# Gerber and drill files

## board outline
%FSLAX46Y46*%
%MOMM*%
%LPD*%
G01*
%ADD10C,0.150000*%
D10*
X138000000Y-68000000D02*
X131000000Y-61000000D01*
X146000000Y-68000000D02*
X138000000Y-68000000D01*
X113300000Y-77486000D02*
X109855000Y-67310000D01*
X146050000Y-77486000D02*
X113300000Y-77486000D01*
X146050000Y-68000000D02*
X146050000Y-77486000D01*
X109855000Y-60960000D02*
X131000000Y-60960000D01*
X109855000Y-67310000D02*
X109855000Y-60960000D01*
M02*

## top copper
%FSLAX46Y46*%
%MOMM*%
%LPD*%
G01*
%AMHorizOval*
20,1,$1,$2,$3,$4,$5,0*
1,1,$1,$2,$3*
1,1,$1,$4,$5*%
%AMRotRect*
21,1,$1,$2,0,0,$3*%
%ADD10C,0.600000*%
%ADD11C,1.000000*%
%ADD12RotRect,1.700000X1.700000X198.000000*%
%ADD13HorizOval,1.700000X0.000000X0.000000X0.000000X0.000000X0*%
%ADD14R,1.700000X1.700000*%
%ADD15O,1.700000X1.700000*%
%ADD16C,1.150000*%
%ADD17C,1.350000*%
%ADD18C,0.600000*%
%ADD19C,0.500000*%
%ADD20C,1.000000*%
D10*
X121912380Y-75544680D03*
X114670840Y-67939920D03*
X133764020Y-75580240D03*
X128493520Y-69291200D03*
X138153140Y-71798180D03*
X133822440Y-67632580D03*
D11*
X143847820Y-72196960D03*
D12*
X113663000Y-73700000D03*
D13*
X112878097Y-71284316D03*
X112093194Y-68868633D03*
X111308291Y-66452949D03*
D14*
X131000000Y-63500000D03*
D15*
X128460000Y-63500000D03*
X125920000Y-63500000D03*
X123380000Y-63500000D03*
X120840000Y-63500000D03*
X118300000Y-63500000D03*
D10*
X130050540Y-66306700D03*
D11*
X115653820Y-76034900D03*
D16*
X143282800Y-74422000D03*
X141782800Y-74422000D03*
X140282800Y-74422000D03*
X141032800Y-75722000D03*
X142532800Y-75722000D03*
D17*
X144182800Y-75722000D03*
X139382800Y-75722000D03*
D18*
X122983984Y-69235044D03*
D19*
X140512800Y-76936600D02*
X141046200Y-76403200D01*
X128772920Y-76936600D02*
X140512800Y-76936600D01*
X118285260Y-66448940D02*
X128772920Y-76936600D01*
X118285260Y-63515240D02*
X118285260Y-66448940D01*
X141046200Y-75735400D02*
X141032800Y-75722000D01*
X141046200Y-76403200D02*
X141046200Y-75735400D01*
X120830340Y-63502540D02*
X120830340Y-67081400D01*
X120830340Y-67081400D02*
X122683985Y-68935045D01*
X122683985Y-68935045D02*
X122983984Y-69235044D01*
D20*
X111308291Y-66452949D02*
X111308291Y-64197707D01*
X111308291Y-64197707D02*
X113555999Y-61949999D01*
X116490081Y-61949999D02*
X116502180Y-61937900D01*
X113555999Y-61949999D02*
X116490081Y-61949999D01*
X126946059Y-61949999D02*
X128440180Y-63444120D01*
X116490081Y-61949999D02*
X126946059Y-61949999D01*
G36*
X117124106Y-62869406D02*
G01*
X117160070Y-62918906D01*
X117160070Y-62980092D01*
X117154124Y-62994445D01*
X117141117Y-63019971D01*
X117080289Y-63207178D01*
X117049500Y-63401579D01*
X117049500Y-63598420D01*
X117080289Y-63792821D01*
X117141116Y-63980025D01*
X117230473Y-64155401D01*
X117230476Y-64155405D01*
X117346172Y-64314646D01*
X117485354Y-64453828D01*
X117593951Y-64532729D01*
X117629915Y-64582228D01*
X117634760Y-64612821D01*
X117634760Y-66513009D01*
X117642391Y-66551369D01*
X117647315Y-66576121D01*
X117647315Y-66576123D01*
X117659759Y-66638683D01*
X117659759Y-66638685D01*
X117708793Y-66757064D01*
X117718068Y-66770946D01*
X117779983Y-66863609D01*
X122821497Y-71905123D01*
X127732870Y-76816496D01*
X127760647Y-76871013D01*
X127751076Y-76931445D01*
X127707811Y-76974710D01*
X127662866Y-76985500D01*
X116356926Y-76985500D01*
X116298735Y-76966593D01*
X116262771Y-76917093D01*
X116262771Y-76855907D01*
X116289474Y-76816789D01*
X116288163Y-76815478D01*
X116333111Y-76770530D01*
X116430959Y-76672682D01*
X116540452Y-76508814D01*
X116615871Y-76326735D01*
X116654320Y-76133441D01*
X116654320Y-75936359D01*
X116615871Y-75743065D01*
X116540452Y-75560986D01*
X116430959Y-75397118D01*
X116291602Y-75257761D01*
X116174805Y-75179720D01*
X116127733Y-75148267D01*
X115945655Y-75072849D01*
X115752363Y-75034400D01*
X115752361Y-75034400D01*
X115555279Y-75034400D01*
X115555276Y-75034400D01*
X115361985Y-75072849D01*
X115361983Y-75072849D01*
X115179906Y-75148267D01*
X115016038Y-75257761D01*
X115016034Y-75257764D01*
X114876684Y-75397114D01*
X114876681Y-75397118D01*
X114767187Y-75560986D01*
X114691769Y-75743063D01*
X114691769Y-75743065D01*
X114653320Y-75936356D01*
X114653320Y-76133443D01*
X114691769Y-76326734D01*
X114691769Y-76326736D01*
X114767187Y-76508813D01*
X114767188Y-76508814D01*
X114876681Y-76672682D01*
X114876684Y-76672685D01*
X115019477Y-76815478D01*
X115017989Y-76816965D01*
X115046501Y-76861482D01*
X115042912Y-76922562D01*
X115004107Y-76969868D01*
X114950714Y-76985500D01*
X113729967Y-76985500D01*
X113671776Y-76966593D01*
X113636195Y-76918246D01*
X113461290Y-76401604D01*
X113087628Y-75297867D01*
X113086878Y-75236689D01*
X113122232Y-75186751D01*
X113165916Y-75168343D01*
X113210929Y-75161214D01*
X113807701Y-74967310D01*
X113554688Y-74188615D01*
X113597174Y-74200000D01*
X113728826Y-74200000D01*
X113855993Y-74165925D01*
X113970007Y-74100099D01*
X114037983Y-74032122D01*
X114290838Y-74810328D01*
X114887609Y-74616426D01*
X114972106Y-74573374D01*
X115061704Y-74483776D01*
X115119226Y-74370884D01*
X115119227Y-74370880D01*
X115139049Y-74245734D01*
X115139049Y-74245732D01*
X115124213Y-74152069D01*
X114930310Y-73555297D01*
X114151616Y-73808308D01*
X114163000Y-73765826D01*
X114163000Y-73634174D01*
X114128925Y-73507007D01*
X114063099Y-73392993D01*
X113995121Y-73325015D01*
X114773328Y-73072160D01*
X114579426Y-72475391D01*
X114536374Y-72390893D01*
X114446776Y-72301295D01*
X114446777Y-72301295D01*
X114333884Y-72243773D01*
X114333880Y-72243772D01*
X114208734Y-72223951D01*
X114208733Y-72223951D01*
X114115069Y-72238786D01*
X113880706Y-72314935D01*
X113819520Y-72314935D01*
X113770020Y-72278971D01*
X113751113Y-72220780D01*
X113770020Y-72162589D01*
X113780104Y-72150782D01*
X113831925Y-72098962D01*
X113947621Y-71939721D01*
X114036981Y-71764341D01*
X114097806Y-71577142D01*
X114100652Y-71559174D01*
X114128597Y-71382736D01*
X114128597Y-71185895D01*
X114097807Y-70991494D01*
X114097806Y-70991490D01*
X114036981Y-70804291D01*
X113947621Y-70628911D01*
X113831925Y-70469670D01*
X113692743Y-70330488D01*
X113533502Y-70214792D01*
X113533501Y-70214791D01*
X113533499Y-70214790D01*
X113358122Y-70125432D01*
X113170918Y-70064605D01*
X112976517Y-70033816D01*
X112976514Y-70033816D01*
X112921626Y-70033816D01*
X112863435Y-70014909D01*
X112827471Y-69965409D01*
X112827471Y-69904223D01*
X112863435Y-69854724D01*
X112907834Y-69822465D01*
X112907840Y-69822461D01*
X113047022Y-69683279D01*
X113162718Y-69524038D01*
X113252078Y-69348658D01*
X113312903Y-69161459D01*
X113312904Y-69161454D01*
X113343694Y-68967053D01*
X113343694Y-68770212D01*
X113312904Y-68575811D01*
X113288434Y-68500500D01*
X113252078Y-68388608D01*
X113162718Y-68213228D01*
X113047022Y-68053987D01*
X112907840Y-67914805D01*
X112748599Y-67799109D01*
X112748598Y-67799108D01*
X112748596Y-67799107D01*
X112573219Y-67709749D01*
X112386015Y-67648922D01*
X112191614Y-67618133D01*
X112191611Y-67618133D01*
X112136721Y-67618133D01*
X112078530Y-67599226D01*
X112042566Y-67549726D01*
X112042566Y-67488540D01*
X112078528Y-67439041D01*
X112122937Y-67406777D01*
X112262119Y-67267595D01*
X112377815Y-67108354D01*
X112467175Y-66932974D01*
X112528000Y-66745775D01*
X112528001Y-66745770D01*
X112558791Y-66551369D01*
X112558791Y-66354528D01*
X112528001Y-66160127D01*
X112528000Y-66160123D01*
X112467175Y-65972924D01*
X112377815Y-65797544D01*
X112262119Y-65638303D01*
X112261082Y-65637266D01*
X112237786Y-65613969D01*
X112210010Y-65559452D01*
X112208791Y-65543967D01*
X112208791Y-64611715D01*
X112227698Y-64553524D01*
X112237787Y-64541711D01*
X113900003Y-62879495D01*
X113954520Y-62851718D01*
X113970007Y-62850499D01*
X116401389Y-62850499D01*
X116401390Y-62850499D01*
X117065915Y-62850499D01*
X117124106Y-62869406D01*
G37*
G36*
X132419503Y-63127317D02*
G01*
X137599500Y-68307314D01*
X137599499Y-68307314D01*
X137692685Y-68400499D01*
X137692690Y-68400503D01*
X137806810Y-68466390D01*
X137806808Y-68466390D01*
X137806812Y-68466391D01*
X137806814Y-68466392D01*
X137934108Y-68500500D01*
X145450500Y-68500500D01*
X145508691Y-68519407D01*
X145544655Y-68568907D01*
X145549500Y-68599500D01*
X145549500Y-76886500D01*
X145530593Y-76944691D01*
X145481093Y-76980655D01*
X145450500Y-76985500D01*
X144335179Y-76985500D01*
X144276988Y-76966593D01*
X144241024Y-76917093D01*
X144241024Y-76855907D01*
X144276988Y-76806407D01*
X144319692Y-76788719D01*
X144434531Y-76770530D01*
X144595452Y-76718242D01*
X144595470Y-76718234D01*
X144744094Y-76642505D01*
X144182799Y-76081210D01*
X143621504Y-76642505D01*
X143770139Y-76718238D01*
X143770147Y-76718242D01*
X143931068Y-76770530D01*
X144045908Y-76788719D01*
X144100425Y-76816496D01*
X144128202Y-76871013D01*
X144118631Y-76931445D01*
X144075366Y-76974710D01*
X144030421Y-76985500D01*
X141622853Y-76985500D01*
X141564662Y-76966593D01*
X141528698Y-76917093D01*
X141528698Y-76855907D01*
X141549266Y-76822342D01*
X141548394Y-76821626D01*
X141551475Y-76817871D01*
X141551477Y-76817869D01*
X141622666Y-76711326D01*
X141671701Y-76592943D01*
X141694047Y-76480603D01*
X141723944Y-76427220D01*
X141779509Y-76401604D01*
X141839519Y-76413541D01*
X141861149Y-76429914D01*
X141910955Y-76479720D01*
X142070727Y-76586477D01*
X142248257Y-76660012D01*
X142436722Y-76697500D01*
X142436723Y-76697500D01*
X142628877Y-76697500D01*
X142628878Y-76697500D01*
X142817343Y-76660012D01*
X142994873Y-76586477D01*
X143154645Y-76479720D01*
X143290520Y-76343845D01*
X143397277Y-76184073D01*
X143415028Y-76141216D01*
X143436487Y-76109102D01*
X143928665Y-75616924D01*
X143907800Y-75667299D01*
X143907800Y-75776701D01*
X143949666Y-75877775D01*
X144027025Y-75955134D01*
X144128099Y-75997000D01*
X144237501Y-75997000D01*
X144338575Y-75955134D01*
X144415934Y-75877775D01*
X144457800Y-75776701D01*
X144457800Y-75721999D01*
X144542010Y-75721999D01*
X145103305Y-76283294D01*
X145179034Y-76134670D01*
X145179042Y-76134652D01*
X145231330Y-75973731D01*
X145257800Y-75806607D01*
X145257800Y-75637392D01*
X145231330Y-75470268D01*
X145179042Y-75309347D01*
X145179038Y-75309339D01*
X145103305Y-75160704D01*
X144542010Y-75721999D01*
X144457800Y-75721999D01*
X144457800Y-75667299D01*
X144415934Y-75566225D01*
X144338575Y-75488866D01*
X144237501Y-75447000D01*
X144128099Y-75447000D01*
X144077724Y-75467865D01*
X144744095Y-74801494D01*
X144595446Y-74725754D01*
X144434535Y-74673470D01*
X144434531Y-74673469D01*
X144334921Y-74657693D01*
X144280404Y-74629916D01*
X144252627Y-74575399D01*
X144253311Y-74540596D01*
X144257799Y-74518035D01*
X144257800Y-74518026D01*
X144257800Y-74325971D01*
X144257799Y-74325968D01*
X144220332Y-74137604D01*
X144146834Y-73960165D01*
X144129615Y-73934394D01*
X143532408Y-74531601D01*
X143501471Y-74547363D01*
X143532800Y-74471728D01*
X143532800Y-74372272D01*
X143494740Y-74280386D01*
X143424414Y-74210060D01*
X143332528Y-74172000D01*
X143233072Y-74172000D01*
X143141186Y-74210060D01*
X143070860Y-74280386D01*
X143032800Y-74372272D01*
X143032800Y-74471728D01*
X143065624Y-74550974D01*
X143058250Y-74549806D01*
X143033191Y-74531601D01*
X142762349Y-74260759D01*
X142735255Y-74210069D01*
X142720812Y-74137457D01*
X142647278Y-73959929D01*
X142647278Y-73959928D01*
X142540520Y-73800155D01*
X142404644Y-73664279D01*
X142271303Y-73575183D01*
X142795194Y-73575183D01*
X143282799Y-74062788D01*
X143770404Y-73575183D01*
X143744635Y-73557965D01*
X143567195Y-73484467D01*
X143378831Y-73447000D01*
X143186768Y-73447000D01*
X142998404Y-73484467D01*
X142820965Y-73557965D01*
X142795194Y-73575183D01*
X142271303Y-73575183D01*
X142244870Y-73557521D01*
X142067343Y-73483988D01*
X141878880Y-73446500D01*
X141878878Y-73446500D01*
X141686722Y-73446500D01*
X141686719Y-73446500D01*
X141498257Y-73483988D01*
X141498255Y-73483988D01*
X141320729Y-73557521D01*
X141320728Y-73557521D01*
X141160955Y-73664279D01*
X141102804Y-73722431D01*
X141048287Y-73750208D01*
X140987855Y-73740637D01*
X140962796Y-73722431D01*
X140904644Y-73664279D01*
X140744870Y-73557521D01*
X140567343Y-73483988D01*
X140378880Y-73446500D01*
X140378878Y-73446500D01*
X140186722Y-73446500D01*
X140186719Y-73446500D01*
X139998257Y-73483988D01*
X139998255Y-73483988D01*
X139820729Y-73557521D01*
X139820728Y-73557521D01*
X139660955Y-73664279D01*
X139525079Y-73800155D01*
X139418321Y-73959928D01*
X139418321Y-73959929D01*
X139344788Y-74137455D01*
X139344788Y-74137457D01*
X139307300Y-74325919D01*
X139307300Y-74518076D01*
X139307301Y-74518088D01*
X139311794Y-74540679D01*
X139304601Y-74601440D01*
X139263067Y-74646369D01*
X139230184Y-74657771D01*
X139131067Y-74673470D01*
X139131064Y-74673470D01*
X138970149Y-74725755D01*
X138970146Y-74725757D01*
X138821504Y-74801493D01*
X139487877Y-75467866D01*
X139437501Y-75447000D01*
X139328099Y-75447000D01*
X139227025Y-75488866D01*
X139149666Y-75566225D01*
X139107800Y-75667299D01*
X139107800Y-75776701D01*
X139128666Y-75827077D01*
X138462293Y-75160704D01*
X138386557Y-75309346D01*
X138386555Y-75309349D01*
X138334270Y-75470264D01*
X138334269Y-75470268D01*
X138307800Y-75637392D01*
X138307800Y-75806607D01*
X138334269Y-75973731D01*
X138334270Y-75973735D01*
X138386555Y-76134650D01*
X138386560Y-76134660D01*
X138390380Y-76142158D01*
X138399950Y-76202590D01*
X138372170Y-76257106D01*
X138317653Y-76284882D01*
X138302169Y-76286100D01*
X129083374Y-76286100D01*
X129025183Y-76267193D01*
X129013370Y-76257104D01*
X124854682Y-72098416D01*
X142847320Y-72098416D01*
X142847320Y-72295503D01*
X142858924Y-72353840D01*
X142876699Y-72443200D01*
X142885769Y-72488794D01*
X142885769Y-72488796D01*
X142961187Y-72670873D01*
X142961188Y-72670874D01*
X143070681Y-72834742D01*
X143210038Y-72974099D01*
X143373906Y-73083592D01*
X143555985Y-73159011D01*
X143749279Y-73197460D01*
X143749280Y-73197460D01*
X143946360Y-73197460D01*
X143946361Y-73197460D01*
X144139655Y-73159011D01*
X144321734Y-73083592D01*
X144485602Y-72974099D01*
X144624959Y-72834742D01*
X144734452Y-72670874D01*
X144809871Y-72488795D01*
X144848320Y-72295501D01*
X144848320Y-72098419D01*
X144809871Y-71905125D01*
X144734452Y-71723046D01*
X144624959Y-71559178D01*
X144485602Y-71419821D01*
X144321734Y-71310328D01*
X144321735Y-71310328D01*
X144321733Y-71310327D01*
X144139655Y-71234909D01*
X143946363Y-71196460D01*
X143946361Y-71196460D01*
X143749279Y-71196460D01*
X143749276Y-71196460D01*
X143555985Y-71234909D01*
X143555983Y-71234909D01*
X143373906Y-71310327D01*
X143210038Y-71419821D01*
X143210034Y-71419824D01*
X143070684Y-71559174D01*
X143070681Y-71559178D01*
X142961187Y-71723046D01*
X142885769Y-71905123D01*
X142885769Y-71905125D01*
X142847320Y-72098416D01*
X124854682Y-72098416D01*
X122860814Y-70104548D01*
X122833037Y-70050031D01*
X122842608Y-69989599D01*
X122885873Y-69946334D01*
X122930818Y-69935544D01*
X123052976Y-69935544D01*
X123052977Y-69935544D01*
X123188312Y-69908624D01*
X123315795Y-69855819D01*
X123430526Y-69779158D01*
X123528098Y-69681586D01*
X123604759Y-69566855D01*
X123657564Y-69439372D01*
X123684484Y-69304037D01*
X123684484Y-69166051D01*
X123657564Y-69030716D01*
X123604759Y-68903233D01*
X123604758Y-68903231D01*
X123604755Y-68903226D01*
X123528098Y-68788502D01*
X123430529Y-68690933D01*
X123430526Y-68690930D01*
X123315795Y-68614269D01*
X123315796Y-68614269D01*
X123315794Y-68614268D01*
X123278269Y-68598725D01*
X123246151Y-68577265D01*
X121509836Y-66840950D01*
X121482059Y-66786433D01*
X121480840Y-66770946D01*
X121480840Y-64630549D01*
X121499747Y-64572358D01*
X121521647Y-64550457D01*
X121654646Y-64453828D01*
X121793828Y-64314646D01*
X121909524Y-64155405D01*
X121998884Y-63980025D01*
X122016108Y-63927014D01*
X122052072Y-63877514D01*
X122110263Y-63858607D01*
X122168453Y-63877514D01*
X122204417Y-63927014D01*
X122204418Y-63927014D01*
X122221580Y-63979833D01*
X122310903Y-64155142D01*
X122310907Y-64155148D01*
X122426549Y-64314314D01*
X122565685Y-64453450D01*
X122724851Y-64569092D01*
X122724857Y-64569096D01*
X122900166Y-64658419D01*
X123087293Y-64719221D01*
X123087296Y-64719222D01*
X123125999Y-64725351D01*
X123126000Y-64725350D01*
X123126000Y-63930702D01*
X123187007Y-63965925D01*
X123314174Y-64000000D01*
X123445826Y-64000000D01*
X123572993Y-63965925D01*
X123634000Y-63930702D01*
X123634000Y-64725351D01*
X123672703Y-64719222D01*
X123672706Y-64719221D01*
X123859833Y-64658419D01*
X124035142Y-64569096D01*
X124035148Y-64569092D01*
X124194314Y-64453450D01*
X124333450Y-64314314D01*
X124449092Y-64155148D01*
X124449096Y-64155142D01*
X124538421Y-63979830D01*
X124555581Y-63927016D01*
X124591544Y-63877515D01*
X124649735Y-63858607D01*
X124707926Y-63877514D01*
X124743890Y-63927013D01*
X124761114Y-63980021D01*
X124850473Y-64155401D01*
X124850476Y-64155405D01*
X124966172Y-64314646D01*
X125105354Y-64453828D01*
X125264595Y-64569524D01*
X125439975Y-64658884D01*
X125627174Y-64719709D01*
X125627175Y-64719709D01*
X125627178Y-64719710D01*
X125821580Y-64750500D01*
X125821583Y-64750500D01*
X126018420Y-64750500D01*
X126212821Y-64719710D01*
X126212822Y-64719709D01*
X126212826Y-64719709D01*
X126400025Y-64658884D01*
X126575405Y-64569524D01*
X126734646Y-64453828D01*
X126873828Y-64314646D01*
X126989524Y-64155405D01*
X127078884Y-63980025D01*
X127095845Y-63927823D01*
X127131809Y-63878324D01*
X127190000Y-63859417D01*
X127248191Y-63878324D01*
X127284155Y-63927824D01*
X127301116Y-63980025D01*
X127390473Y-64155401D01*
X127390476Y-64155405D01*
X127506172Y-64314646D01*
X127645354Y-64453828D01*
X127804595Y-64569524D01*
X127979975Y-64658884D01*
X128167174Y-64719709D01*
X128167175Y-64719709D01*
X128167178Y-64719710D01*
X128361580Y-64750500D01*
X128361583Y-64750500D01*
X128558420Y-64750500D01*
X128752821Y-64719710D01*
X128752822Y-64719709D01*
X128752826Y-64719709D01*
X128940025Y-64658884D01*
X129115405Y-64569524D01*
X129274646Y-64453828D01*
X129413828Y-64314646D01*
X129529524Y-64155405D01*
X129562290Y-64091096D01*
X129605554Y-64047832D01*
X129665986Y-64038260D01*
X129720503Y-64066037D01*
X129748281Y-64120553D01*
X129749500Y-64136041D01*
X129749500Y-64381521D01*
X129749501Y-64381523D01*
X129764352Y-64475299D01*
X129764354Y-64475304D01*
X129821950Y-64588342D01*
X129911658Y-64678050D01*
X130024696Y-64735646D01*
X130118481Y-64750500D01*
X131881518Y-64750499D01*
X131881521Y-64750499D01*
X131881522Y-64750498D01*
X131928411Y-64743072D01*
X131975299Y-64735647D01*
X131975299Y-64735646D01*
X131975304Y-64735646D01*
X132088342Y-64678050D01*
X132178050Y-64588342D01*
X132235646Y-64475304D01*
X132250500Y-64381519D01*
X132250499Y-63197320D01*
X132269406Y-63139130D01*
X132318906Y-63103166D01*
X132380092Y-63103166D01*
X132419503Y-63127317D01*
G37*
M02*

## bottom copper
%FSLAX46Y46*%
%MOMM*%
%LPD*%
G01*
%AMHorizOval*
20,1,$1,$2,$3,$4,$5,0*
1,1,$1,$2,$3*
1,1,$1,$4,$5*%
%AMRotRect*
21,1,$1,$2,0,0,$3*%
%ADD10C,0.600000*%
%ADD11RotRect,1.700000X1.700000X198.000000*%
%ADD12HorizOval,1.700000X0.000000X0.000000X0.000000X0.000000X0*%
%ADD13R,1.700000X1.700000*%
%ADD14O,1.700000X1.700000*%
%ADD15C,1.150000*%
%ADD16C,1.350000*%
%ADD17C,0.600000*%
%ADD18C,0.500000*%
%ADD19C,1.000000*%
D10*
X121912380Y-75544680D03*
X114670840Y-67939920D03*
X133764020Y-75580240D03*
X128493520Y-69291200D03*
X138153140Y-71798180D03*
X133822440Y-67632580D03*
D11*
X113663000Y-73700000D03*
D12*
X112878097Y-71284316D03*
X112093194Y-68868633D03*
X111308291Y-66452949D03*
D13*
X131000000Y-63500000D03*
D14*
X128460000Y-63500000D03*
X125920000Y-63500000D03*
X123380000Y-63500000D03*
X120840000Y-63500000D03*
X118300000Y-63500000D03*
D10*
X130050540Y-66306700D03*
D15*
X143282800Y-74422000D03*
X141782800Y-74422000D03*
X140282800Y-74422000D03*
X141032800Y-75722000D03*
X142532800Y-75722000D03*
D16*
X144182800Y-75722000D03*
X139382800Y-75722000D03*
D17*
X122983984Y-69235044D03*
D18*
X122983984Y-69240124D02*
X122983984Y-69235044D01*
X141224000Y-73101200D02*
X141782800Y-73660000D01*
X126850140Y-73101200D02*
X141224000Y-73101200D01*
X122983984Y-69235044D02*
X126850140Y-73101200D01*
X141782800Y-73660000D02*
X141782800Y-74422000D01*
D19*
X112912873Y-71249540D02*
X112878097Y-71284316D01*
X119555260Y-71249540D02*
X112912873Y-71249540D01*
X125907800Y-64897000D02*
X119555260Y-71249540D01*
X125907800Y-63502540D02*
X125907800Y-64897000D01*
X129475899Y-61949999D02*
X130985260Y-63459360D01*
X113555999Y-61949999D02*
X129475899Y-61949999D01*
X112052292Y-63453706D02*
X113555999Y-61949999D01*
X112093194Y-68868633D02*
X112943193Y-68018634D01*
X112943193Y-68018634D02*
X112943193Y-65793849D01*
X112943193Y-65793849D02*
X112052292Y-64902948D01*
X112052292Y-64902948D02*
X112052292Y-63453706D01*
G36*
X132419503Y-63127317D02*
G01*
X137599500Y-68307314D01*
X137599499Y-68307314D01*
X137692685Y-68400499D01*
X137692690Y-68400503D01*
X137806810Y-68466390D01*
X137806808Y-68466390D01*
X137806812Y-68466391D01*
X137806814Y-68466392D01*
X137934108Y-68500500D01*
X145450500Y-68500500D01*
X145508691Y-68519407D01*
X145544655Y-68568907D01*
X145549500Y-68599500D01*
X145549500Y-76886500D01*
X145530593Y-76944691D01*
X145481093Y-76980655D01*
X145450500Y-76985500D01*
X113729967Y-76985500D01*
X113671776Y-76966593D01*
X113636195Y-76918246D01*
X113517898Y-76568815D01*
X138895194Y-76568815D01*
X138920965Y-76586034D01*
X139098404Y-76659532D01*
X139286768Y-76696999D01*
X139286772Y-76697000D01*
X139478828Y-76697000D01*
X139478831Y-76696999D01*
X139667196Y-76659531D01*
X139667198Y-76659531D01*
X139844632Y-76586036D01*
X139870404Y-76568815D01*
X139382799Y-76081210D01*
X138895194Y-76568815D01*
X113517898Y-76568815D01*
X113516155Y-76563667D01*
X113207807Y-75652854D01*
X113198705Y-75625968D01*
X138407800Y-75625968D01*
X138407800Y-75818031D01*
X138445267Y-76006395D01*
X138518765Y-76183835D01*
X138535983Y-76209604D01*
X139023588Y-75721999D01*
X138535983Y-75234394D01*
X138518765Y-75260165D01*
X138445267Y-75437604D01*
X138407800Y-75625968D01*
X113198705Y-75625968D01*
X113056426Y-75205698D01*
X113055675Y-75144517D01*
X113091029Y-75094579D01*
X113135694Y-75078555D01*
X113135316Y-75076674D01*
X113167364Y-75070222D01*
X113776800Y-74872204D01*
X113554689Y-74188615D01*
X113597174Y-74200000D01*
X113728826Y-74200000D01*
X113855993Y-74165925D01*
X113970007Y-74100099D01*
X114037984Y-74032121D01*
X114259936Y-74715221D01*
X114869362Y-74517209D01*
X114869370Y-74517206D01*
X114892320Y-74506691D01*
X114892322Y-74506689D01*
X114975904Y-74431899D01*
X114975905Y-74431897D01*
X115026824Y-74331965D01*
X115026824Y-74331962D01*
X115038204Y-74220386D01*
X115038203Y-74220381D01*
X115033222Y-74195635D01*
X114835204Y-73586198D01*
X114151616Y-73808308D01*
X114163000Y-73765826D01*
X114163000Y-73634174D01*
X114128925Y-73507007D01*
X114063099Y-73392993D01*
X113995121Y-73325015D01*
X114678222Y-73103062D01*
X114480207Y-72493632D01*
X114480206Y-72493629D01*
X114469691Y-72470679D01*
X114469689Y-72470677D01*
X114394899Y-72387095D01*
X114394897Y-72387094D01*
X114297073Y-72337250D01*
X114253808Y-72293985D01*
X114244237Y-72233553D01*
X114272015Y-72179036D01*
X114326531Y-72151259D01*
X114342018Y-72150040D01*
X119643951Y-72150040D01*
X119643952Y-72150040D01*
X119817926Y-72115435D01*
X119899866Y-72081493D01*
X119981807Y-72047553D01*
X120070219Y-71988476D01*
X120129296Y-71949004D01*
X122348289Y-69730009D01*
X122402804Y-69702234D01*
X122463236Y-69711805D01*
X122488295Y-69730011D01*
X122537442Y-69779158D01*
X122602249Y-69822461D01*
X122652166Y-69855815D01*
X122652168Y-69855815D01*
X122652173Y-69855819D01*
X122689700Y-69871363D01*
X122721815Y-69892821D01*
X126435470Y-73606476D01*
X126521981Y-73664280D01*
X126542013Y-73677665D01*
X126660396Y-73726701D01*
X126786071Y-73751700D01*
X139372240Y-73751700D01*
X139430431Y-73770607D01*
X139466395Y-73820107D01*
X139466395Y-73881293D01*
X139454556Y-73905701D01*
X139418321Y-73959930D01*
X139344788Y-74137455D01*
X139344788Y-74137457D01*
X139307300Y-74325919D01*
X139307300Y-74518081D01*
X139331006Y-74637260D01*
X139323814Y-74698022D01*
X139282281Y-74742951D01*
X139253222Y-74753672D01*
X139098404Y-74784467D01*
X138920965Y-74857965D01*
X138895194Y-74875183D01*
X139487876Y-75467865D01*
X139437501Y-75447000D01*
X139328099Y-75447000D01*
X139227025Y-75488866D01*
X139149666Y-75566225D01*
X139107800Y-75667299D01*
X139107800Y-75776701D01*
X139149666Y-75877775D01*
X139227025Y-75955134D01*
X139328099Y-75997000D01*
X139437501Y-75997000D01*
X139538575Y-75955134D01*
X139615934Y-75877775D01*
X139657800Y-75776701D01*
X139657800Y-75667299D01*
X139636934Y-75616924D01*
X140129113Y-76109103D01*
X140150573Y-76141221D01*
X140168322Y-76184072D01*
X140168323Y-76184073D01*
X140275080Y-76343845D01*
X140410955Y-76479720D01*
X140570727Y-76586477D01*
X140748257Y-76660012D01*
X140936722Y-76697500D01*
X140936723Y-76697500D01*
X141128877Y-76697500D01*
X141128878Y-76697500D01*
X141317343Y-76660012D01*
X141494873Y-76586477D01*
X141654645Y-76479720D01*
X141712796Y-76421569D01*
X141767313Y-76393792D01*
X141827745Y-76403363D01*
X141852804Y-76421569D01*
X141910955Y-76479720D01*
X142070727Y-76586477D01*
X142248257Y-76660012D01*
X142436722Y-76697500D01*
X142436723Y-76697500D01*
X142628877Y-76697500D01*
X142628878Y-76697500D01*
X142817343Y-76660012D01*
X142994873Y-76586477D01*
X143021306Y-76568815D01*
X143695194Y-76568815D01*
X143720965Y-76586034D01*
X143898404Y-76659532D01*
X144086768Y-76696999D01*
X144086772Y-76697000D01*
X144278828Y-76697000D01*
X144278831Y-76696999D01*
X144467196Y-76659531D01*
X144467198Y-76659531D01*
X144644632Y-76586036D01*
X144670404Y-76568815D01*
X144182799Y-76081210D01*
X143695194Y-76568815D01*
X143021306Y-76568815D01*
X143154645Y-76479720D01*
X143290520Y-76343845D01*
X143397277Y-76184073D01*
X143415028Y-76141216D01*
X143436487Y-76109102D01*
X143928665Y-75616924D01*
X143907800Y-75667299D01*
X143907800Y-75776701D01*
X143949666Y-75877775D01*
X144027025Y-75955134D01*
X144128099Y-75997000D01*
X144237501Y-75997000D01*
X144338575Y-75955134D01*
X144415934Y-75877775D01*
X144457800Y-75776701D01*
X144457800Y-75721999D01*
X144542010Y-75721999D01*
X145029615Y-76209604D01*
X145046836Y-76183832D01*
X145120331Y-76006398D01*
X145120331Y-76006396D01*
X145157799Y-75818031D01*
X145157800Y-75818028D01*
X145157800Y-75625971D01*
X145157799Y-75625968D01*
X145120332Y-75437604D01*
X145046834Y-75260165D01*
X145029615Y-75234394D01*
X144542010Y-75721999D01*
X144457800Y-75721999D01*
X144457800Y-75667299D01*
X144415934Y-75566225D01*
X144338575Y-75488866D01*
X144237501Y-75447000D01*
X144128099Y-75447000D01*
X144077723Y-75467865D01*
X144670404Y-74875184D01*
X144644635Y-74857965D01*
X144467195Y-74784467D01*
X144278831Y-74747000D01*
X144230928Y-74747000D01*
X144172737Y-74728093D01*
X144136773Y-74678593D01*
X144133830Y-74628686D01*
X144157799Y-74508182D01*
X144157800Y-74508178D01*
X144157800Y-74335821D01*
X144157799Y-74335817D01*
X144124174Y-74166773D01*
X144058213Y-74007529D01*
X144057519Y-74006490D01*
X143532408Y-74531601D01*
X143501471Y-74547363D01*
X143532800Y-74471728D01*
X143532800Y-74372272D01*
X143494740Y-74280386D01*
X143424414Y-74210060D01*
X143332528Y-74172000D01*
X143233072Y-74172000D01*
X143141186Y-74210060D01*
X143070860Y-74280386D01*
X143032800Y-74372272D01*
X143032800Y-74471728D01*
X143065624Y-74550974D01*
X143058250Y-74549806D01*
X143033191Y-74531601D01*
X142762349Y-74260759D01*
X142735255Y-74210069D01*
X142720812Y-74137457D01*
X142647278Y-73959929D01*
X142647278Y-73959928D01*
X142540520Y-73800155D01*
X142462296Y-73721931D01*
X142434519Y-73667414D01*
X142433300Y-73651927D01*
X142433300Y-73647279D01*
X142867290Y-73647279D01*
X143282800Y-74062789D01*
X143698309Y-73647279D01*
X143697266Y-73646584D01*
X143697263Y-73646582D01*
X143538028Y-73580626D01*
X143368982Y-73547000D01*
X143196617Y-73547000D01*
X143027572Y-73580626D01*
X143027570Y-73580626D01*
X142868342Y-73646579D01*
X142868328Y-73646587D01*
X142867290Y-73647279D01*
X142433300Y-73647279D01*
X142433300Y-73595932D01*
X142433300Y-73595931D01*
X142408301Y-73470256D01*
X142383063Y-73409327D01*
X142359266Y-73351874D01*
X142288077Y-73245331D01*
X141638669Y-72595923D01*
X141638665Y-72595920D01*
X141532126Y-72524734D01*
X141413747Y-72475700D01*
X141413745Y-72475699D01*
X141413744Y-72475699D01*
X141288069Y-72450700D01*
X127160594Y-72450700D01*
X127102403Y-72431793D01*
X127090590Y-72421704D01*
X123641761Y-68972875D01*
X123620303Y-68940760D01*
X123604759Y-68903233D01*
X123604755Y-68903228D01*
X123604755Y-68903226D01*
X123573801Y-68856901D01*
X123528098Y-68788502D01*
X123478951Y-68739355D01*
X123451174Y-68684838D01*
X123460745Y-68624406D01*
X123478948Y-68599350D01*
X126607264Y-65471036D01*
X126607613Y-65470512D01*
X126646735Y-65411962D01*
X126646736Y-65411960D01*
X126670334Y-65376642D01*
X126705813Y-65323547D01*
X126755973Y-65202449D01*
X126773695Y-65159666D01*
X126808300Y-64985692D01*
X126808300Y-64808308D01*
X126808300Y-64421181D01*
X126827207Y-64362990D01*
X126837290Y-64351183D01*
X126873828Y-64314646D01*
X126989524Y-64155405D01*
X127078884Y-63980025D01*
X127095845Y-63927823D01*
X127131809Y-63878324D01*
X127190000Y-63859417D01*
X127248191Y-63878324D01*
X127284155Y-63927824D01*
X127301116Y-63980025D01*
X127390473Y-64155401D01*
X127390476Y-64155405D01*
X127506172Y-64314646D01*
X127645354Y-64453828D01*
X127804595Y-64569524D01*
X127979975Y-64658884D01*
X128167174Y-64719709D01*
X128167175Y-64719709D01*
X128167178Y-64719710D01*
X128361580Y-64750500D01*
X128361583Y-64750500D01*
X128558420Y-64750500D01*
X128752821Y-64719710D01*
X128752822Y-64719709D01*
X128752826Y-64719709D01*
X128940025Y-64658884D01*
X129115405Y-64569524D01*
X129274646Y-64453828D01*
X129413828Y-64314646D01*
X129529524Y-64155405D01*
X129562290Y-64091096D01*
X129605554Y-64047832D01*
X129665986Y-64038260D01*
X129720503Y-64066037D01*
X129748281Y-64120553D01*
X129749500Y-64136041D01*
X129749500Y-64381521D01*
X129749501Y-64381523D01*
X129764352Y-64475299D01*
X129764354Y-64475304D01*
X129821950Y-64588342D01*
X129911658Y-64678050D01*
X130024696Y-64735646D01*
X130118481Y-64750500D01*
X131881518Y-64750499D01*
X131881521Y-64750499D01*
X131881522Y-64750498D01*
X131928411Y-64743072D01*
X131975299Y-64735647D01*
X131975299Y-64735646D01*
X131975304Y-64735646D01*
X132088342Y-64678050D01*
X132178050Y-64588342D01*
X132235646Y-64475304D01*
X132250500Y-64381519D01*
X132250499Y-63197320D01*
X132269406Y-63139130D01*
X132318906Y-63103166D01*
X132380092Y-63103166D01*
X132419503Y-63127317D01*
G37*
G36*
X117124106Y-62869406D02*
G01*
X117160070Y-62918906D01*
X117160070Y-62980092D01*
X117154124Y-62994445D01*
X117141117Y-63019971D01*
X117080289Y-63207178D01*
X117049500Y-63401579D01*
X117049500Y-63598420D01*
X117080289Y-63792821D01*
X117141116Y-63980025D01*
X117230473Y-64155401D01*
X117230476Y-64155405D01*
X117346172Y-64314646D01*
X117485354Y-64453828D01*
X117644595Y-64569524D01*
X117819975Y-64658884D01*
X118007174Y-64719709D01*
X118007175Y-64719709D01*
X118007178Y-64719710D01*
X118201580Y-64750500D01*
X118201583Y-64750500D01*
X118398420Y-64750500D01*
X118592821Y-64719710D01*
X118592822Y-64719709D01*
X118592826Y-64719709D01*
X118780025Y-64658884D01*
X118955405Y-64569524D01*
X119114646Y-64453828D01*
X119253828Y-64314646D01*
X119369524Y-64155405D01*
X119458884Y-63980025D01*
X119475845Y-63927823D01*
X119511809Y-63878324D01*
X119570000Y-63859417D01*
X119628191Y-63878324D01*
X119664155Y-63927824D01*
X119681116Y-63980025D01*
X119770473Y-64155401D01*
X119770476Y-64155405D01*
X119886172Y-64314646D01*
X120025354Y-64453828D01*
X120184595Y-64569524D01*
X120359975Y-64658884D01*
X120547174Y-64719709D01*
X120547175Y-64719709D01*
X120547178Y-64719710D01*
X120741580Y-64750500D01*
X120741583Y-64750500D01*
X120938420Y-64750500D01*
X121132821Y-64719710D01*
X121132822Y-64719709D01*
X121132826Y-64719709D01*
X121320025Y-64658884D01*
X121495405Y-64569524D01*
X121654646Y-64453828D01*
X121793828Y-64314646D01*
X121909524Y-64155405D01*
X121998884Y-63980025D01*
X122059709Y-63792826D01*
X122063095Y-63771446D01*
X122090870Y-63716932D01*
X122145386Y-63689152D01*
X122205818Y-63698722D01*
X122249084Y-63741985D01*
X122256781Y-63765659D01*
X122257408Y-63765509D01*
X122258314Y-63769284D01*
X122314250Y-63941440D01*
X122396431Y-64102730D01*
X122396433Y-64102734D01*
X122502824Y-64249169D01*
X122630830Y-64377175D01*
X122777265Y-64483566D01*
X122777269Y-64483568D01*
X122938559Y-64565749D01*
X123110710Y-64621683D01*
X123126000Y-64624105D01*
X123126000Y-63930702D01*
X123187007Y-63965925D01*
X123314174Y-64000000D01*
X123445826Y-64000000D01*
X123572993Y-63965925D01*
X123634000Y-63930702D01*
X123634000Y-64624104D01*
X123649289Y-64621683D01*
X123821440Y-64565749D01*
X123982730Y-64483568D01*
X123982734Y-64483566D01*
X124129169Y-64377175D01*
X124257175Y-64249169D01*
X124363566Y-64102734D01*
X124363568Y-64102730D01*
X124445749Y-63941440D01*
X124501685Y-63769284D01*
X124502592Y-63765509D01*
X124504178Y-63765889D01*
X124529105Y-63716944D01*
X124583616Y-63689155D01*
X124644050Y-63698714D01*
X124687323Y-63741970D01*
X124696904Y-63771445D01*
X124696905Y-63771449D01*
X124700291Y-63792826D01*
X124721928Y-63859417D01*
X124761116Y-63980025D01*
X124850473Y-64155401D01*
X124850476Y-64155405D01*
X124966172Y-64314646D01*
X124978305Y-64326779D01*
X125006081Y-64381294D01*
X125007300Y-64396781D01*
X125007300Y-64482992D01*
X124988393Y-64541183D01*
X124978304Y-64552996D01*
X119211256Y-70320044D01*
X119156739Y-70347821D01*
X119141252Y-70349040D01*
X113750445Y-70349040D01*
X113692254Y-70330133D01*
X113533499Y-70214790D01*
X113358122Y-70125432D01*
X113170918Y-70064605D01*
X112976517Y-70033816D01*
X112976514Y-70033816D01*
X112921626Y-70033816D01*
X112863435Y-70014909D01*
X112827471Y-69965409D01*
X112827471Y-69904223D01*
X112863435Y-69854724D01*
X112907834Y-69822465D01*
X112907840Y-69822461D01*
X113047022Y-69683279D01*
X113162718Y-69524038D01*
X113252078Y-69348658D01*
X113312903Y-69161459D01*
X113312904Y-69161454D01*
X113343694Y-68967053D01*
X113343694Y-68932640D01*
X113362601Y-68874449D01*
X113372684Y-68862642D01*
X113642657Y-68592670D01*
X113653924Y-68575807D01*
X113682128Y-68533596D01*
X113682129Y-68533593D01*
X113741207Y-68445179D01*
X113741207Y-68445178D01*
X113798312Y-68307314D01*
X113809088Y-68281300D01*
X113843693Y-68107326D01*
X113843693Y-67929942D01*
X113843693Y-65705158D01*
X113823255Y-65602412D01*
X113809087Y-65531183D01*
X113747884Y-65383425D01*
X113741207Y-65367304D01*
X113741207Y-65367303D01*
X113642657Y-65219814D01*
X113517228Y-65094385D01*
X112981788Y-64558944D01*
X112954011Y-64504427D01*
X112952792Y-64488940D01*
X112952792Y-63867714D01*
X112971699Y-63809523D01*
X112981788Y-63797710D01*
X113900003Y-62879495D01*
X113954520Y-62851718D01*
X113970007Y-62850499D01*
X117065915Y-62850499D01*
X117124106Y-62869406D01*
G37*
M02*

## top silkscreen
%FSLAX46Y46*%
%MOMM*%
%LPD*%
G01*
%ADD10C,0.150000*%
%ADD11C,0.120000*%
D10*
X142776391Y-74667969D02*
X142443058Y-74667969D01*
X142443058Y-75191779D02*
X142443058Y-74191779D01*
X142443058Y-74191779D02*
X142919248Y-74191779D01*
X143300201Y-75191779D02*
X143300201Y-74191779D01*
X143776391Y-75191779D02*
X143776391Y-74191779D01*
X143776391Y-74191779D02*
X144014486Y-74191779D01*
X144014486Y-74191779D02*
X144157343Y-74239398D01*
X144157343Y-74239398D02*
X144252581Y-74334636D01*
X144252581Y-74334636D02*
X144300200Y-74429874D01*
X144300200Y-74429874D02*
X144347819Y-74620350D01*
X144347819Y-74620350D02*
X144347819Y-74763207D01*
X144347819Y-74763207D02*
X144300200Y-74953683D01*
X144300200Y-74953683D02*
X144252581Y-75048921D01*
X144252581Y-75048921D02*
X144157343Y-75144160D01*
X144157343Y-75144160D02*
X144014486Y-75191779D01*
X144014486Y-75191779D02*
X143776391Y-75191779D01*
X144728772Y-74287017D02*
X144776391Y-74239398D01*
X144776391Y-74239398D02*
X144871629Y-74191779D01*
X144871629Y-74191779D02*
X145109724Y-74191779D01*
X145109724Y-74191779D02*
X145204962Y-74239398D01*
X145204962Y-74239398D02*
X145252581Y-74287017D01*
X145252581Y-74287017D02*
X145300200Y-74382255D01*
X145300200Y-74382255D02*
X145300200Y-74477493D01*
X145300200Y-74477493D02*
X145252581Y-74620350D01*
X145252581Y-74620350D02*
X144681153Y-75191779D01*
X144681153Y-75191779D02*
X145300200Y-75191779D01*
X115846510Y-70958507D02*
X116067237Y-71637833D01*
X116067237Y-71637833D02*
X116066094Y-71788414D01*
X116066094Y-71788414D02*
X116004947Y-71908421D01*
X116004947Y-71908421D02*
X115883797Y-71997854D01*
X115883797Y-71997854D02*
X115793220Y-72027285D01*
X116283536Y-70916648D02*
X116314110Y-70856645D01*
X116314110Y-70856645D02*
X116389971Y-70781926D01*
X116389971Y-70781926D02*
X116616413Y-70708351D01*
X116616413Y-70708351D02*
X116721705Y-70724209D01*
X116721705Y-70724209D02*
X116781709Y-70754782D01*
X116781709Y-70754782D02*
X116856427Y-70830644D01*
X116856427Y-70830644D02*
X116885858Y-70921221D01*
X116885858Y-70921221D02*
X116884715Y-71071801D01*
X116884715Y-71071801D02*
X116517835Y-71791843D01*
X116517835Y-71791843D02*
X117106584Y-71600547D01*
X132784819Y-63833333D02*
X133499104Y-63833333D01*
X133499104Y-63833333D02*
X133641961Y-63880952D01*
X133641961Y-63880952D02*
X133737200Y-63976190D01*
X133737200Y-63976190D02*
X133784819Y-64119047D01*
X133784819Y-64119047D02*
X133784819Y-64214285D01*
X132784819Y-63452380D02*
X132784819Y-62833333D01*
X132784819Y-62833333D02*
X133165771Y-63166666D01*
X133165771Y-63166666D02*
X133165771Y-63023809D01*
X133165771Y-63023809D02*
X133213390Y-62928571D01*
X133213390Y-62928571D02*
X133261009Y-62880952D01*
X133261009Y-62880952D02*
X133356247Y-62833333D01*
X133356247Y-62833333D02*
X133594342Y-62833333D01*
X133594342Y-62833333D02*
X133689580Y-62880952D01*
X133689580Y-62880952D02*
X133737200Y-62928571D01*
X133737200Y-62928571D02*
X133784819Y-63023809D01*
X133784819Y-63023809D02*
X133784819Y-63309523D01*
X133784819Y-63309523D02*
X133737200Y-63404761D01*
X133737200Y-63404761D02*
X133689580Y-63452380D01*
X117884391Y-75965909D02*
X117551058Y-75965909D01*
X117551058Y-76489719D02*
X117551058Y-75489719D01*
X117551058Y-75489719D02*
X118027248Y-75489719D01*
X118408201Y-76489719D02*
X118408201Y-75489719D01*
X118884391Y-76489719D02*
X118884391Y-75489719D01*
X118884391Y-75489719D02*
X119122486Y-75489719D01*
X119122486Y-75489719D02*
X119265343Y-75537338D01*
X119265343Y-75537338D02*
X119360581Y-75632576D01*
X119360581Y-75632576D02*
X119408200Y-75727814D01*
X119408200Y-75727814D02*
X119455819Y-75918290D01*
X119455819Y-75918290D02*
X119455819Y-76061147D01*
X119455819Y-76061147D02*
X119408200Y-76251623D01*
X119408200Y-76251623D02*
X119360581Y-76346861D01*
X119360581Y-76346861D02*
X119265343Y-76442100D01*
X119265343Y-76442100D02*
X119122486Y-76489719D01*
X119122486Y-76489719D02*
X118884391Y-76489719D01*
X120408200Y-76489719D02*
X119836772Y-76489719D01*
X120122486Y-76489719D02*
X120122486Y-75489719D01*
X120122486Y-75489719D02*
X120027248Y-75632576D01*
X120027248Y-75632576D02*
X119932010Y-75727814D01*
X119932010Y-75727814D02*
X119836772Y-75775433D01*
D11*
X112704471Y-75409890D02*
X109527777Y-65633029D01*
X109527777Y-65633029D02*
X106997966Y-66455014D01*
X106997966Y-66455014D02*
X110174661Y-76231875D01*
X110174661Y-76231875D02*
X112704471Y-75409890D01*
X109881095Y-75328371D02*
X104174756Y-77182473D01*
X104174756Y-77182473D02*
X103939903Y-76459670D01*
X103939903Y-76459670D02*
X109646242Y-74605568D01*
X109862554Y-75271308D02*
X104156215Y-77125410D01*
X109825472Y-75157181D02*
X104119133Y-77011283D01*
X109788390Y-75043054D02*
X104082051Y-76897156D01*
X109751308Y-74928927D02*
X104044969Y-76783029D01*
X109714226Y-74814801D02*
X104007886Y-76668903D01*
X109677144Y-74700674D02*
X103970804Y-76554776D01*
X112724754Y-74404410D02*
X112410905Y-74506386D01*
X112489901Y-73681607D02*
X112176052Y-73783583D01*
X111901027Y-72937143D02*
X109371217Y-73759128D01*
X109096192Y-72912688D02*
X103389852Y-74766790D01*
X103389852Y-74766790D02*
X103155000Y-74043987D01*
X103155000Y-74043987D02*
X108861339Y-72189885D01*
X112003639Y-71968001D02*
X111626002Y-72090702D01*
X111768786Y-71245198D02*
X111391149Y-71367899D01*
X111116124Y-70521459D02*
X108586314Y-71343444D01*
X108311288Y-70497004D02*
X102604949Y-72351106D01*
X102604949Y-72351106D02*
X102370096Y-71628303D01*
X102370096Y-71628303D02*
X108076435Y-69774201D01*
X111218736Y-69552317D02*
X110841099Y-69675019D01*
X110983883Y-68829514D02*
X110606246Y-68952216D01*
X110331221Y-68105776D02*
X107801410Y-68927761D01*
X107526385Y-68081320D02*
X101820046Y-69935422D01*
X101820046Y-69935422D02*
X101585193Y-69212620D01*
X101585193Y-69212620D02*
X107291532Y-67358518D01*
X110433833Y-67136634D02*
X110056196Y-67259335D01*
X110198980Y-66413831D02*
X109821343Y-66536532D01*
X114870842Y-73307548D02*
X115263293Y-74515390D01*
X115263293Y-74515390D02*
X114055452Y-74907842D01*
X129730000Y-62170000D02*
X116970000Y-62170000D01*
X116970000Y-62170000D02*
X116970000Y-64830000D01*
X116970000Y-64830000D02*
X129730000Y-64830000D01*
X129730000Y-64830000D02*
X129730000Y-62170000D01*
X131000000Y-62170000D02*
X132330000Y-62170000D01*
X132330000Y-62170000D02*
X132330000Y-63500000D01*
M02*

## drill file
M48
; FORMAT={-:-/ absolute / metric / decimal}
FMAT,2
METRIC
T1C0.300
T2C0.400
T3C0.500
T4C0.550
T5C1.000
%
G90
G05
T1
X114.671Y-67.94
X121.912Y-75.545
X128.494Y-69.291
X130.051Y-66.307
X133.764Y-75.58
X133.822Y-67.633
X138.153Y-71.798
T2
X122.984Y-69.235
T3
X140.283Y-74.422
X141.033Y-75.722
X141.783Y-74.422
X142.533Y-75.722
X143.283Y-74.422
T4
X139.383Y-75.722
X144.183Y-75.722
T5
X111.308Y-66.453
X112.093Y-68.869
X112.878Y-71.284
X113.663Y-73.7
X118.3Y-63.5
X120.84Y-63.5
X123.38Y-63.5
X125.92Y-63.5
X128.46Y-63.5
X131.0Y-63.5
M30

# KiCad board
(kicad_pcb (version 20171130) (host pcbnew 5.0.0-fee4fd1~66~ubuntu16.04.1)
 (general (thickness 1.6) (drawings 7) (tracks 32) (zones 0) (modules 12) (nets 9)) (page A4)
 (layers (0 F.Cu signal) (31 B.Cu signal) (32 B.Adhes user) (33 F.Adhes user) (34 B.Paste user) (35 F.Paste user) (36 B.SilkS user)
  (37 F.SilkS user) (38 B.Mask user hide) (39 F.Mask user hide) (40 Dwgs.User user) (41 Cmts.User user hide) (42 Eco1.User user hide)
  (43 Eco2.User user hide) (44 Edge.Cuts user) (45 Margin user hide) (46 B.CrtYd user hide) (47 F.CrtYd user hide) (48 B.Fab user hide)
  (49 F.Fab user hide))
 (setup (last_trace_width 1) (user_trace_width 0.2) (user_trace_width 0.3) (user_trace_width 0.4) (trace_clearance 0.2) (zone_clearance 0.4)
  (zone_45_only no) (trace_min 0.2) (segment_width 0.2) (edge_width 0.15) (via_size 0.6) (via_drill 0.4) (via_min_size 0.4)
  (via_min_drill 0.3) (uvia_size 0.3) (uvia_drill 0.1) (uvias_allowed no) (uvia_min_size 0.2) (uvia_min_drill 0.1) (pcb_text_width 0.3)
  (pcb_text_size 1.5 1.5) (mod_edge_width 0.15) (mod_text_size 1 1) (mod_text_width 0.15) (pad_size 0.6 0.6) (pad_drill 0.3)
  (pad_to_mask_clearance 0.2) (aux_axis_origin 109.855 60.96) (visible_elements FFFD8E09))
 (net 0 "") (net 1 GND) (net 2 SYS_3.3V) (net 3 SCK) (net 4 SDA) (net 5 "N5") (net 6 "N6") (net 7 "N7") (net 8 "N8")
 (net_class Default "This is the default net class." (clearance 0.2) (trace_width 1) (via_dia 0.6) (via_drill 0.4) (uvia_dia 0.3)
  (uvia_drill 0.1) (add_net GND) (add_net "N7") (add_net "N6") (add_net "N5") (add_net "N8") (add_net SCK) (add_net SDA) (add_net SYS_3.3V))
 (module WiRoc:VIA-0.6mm (layer F.Cu) (at 121.91238 75.54468)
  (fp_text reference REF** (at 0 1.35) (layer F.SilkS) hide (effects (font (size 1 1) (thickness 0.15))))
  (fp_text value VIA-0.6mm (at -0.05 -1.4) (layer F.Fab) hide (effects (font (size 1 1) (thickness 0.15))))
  (pad 1 thru_hole circle (at 0 0) (size 0.6 0.6) (drill 0.3) (layers *.Cu) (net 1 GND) (zone_connect 2)))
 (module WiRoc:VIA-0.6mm (layer F.Cu) (at 114.67084 67.93992)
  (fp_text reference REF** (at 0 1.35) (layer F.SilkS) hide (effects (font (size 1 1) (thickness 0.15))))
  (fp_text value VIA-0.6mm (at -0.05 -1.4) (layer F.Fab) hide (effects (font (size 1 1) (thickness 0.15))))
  (pad 1 thru_hole circle (at 0 0) (size 0.6 0.6) (drill 0.3) (layers *.Cu) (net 1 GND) (zone_connect 2)))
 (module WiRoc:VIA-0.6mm (layer F.Cu) (at 133.76402 75.58024)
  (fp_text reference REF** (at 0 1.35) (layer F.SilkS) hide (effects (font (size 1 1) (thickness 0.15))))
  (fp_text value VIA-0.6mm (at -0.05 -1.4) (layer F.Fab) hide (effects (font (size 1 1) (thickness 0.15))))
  (pad 1 thru_hole circle (at 0 0) (size 0.6 0.6) (drill 0.3) (layers *.Cu) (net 1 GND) (zone_connect 2)))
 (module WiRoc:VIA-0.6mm (layer F.Cu) (at 128.49352 69.2912)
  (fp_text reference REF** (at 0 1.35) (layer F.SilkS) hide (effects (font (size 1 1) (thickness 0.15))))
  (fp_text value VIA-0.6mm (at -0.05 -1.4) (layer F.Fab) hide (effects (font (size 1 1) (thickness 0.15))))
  (pad 1 thru_hole circle (at 0 0) (size 0.6 0.6) (drill 0.3) (layers *.Cu) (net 1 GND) (zone_connect 2)))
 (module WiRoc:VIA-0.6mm (layer F.Cu) (at 138.15314 71.79818)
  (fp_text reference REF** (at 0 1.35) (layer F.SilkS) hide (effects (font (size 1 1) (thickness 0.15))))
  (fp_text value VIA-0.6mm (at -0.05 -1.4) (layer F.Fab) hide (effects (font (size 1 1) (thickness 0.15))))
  (pad 1 thru_hole circle (at 0 0) (size 0.6 0.6) (drill 0.3) (layers *.Cu) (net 1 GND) (zone_connect 2)))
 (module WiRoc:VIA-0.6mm (layer F.Cu) (at 133.82244 67.63258)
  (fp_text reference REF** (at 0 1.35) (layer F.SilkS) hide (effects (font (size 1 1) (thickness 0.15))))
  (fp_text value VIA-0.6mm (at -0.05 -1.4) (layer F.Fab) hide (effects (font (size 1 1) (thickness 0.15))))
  (pad 1 thru_hole circle (at 0 0) (size 0.6 0.6) (drill 0.3) (layers *.Cu) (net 1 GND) (zone_connect 2)))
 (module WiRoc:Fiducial (layer F.Cu) (at 143.84782 72.19696)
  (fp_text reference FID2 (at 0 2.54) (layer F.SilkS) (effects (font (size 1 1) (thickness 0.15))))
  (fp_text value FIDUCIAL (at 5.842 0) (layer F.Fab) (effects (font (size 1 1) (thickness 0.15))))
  (pad 1 smd circle (at 0 0) (size 1 1) (layers F.Cu F.Mask) (solder_mask_margin 0.5) (clearance 0.5)))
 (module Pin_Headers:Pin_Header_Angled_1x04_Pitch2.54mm (layer F.Cu) (at 113.663 73.7 198)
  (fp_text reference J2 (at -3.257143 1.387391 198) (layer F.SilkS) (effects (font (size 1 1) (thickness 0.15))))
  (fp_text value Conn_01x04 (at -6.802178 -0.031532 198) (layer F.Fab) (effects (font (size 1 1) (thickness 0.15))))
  (fp_line (start 1.44 -1.33) (end 1.44 8.95) (layer F.SilkS) (width 0.12))
  (fp_line (start 1.44 8.95) (end 4.1 8.95) (layer F.SilkS) (width 0.12))
  (fp_line (start 4.1 8.95) (end 4.1 -1.33) (layer F.SilkS) (width 0.12))
  (fp_line (start 4.1 -1.33) (end 1.44 -1.33) (layer F.SilkS) (width 0.12))
  (fp_line (start 4.1 -0.38) (end 10.1 -0.38) (layer F.SilkS) (width 0.12))
  (fp_line (start 10.1 -0.38) (end 10.1 0.38) (layer F.SilkS) (width 0.12))
  (fp_line (start 10.1 0.38) (end 4.1 0.38) (layer F.SilkS) (width 0.12))
  (fp_line (start 4.1 -0.32) (end 10.1 -0.32) (layer F.SilkS) (width 0.12))
  (fp_line (start 4.1 -0.2) (end 10.1 -0.2) (layer F.SilkS) (width 0.12))
  (fp_line (start 4.1 -0.08) (end 10.1 -0.08) (layer F.SilkS) (width 0.12))
  (fp_line (start 4.1 0.04) (end 10.1 0.04) (layer F.SilkS) (width 0.12))
  (fp_line (start 4.1 0.16) (end 10.1 0.16) (layer F.SilkS) (width 0.12))
  (fp_line (start 4.1 0.28) (end 10.1 0.28) (layer F.SilkS) (width 0.12))
  (fp_line (start 1.11 -0.38) (end 1.44 -0.38) (layer F.SilkS) (width 0.12))
  (fp_line (start 1.11 0.38) (end 1.44 0.38) (layer F.SilkS) (width 0.12))
  (fp_line (start 1.44 1.27) (end 4.1 1.27) (layer F.SilkS) (width 0.12))
  (fp_line (start 4.1 2.16) (end 10.1 2.16) (layer F.SilkS) (width 0.12))
  (fp_line (start 10.1 2.16) (end 10.1 2.92) (layer F.SilkS) (width 0.12))
  (fp_line (start 10.1 2.92) (end 4.1 2.92) (layer F.SilkS) (width 0.12))
  (fp_line (start 1.042929 2.16) (end 1.44 2.16) (layer F.SilkS) (width 0.12))
  (fp_line (start 1.042929 2.92) (end 1.44 2.92) (layer F.SilkS) (width 0.12))
  (fp_line (start 1.44 3.81) (end 4.1 3.81) (layer F.SilkS) (width 0.12))
  (fp_line (start 4.1 4.7) (end 10.1 4.7) (layer F.SilkS) (width 0.12))
  (fp_line (start 10.1 4.7) (end 10.1 5.46) (layer F.SilkS) (width 0.12))
  (fp_line (start 10.1 5.46) (end 4.1 5.46) (layer F.SilkS) (width 0.12))
  (fp_line (start 1.042929 4.7) (end 1.44 4.7) (layer F.SilkS) (width 0.12))
  (fp_line (start 1.042929 5.46) (end 1.44 5.46) (layer F.SilkS) (width 0.12))
  (fp_line (start 1.44 6.35) (end 4.1 6.35) (layer F.SilkS) (width 0.12))
  (fp_line (start 4.1 7.24) (end 10.1 7.24) (layer F.SilkS) (width 0.12))
  (fp_line (start 10.1 7.24) (end 10.1 8) (layer F.SilkS) (width 0.12))
  (fp_line (start 10.1 8) (end 4.1 8) (layer F.SilkS) (width 0.12))
  (fp_line (start 1.042929 7.24) (end 1.44 7.24) (layer F.SilkS) (width 0.12))
  (fp_line (start 1.042929 8) (end 1.44 8) (layer F.SilkS) (width 0.12))
  (fp_line (start -1.27 0) (end -1.27 -1.27) (layer F.SilkS) (width 0.12))
  (fp_line (start -1.27 -1.27) (end 0 -1.27) (layer F.SilkS) (width 0.12))
  (pad 1 thru_hole rect (at 0 0 198) (size 1.7 1.7) (drill 1) (layers *.Cu *.Mask) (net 1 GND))
  (pad 2 thru_hole oval (at 0 2.54 198) (size 1.7 1.7) (drill 1) (layers *.Cu *.Mask) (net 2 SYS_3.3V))
  (pad 3 thru_hole oval (at 0 5.08 198) (size 1.7 1.7) (drill 1) (layers *.Cu *.Mask) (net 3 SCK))
  (pad 4 thru_hole oval (at -0.000001 7.62 198) (size 1.7 1.7) (drill 1) (layers *.Cu *.Mask) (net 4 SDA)))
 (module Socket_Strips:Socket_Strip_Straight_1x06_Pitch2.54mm (layer F.Cu) (at 131 63.5 270)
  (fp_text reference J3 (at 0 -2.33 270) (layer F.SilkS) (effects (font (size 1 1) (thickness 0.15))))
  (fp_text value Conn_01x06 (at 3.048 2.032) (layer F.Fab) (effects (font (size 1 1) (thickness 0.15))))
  (fp_line (start -1.33 1.27) (end -1.33 14.03) (layer F.SilkS) (width 0.12))
  (fp_line (start -1.33 14.03) (end 1.33 14.03) (layer F.SilkS) (width 0.12))
  (fp_line (start 1.33 14.03) (end 1.33 1.27) (layer F.SilkS) (width 0.12))
  (fp_line (start 1.33 1.27) (end -1.33 1.27) (layer F.SilkS) (width 0.12))
  (fp_line (start -1.33 0) (end -1.33 -1.33) (layer F.SilkS) (width 0.12))
  (fp_line (start -1.33 -1.33) (end 0 -1.33) (layer F.SilkS) (width 0.12))
  (pad 1 thru_hole rect (at 0 0 270) (size 1.7 1.7) (drill 1) (layers *.Cu *.Mask) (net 3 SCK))
  (pad 2 thru_hole oval (at 0 2.54 270) (size 1.7 1.7) (drill 1) (layers *.Cu *.Mask) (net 4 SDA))
  (pad 3 thru_hole oval (at 0 5.08 270) (size 1.7 1.7) (drill 1) (layers *.Cu *.Mask) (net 2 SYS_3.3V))
  (pad 4 thru_hole oval (at 0 7.62 270) (size 1.7 1.7) (drill 1) (layers *.Cu *.Mask) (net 1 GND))
  (pad 5 thru_hole oval (at 0 10.16 270) (size 1.7 1.7) (drill 1) (layers *.Cu *.Mask) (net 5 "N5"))
  (pad 6 thru_hole oval (at 0 12.7 270) (size 1.7 1.7) (drill 1) (layers *.Cu *.Mask) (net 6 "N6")))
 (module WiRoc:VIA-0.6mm (layer F.Cu) (at 130.05054 66.3067)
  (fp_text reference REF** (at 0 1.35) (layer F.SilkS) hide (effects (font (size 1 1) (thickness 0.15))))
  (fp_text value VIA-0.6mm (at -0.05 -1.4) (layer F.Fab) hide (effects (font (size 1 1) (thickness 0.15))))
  (pad 1 thru_hole circle (at 0 0) (size 0.6 0.6) (drill 0.3) (layers *.Cu) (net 1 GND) (zone_connect 2)))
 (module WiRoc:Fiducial (layer F.Cu) (at 115.65382 76.0349)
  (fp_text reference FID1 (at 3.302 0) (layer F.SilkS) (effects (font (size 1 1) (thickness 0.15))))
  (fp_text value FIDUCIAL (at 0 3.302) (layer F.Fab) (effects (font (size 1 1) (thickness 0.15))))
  (pad 1 smd circle (at 0 0) (size 1 1) (layers F.Cu F.Mask) (solder_mask_margin 0.5) (clearance 0.5)))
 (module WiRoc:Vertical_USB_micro (layer B.Cu) (at 141.7828 75.072 180)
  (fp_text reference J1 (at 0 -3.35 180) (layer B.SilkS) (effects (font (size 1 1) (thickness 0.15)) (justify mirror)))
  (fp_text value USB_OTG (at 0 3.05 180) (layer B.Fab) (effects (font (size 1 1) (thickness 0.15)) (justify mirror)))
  (pad 5 thru_hole circle (at -1.5 0.65 180) (size 1.15 1.15) (drill 0.5) (layers *.Cu *.Mask) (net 1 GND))
  (pad 3 thru_hole circle (at 0 0.65 180) (size 1.15 1.15) (drill 0.5) (layers *.Cu *.Mask) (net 5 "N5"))
  (pad 1 thru_hole circle (at 1.5 0.65 180) (size 1.15 1.15) (drill 0.5) (layers *.Cu *.Mask) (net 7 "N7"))
  (pad 2 thru_hole circle (at 0.75 -0.65 180) (size 1.15 1.15) (drill 0.5) (layers *.Cu *.Mask) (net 6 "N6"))
  (pad 4 thru_hole circle (at -0.75 -0.65 180) (size 1.15 1.15) (drill 0.5) (layers *.Cu *.Mask) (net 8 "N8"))
  (pad 6 thru_hole circle (at -2.4 -0.65 180) (size 1.35 1.35) (drill 0.55) (layers *.Cu *.Mask) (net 1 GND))
  (pad 6 thru_hole circle (at 2.4 -0.65 180) (size 1.35 1.35) (drill 0.55) (layers *.Cu *.Mask) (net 1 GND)))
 (gr_line (start 138 68) (end 131 61) (layer Edge.Cuts) (width 0.15))
 (gr_line (start 146 68) (end 138 68) (layer Edge.Cuts) (width 0.15))
 (gr_line (start 113.3 77.486) (end 109.855 67.31) (layer Edge.Cuts) (width 0.15))
 (gr_line (start 146.05 77.486) (end 113.3 77.486) (layer Edge.Cuts) (width 0.15))
 (gr_line (start 146.05 68) (end 146.05 77.486) (layer Edge.Cuts) (width 0.15))
 (gr_line (start 109.855 60.96) (end 131 60.96) (layer Edge.Cuts) (width 0.15))
 (gr_line (start 109.855 67.31) (end 109.855 60.96) (layer Edge.Cuts) (width 0.15))
 (segment (start 140.5128 76.9366) (end 141.0462 76.4032) (width 0.5) (layer F.Cu) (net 6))
 (segment (start 128.77292 76.9366) (end 140.5128 76.9366) (width 0.5) (layer F.Cu) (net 6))
 (segment (start 118.28526 66.44894) (end 128.77292 76.9366) (width 0.5) (layer F.Cu) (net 6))
 (segment (start 118.28526 63.51524) (end 118.28526 66.44894) (width 0.5) (layer F.Cu) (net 6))
 (segment (start 141.0462 75.7354) (end 141.0328 75.722) (width 0.5) (layer F.Cu) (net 6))
 (segment (start 141.0462 76.4032) (end 141.0462 75.7354) (width 0.5) (layer F.Cu) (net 6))
 (segment (start 120.83034 63.50254) (end 120.83034 67.0814) (width 0.5) (layer F.Cu) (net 5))
 (segment (start 120.83034 67.0814) (end 122.683985 68.935045) (width 0.5) (layer F.Cu) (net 5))
 (segment (start 122.683985 68.935045) (end 122.983984 69.235044) (width 0.5) (layer F.Cu) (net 5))
 (segment (start 122.983984 69.240124) (end 122.983984 69.235044) (width 0.5) (layer B.Cu) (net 5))
 (via (at 122.983984 69.235044) (size 0.6) (drill 0.4) (layers F.Cu B.Cu) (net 5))
 (segment (start 141.224 73.1012) (end 141.7828 73.66) (width 0.5) (layer B.Cu) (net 5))
 (segment (start 126.85014 73.1012) (end 141.224 73.1012) (width 0.5) (layer B.Cu) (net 5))
 (segment (start 122.983984 69.235044) (end 126.85014 73.1012) (width 0.5) (layer B.Cu) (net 5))
 (segment (start 141.7828 73.66) (end 141.7828 74.422) (width 0.5) (layer B.Cu) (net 5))
 (segment (start 112.912873 71.24954) (end 112.878097 71.284316) (width 1) (layer B.Cu) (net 2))
 (segment (start 119.55526 71.24954) (end 112.912873 71.24954) (width 1) (layer B.Cu) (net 2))
 (segment (start 125.9078 64.897) (end 119.55526 71.24954) (width 1) (layer B.Cu) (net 2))
 (segment (start 125.9078 63.50254) (end 125.9078 64.897) (width 1) (layer B.Cu) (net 2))
 (segment (start 129.475899 61.949999) (end 130.98526 63.45936) (width 1) (layer B.Cu) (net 3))
 (segment (start 113.555999 61.949999) (end 129.475899 61.949999) (width 1) (layer B.Cu) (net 3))
 (segment (start 112.052292 63.453706) (end 113.555999 61.949999) (width 1) (layer B.Cu) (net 3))
 (segment (start 112.093194 68.868633) (end 112.943193 68.018634) (width 1) (layer B.Cu) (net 3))
 (segment (start 112.943193 68.018634) (end 112.943193 65.793849) (width 1) (layer B.Cu) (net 3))
 (segment (start 112.943193 65.793849) (end 112.052292 64.902948) (width 1) (layer B.Cu) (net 3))
 (segment (start 112.052292 64.902948) (end 112.052292 63.453706) (width 1) (layer B.Cu) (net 3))
 (segment (start 111.308291 66.452949) (end 111.308291 64.197707) (width 1) (layer F.Cu) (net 4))
 (segment (start 111.308291 64.197707) (end 113.555999 61.949999) (width 1) (layer F.Cu) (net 4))
 (segment (start 116.490081 61.949999) (end 116.50218 61.9379) (width 1) (layer F.Cu) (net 4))
 (segment (start 113.555999 61.949999) (end 116.490081 61.949999) (width 1) (layer F.Cu) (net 4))
 (segment (start 126.946059 61.949999) (end 128.44018 63.44412) (width 1) (layer F.Cu) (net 4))
 (segment (start 116.490081 61.949999) (end 126.946059 61.949999) (width 1) (layer F.Cu) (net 4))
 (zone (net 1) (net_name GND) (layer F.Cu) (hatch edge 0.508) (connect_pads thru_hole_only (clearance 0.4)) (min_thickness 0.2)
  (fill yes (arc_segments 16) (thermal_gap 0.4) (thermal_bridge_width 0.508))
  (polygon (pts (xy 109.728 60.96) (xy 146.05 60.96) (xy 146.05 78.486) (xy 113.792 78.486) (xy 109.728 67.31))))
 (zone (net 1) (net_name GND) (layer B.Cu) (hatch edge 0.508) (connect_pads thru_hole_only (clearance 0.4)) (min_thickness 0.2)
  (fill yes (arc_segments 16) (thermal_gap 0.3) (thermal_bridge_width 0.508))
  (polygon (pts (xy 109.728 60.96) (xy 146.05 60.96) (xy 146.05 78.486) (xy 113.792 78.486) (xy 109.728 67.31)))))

